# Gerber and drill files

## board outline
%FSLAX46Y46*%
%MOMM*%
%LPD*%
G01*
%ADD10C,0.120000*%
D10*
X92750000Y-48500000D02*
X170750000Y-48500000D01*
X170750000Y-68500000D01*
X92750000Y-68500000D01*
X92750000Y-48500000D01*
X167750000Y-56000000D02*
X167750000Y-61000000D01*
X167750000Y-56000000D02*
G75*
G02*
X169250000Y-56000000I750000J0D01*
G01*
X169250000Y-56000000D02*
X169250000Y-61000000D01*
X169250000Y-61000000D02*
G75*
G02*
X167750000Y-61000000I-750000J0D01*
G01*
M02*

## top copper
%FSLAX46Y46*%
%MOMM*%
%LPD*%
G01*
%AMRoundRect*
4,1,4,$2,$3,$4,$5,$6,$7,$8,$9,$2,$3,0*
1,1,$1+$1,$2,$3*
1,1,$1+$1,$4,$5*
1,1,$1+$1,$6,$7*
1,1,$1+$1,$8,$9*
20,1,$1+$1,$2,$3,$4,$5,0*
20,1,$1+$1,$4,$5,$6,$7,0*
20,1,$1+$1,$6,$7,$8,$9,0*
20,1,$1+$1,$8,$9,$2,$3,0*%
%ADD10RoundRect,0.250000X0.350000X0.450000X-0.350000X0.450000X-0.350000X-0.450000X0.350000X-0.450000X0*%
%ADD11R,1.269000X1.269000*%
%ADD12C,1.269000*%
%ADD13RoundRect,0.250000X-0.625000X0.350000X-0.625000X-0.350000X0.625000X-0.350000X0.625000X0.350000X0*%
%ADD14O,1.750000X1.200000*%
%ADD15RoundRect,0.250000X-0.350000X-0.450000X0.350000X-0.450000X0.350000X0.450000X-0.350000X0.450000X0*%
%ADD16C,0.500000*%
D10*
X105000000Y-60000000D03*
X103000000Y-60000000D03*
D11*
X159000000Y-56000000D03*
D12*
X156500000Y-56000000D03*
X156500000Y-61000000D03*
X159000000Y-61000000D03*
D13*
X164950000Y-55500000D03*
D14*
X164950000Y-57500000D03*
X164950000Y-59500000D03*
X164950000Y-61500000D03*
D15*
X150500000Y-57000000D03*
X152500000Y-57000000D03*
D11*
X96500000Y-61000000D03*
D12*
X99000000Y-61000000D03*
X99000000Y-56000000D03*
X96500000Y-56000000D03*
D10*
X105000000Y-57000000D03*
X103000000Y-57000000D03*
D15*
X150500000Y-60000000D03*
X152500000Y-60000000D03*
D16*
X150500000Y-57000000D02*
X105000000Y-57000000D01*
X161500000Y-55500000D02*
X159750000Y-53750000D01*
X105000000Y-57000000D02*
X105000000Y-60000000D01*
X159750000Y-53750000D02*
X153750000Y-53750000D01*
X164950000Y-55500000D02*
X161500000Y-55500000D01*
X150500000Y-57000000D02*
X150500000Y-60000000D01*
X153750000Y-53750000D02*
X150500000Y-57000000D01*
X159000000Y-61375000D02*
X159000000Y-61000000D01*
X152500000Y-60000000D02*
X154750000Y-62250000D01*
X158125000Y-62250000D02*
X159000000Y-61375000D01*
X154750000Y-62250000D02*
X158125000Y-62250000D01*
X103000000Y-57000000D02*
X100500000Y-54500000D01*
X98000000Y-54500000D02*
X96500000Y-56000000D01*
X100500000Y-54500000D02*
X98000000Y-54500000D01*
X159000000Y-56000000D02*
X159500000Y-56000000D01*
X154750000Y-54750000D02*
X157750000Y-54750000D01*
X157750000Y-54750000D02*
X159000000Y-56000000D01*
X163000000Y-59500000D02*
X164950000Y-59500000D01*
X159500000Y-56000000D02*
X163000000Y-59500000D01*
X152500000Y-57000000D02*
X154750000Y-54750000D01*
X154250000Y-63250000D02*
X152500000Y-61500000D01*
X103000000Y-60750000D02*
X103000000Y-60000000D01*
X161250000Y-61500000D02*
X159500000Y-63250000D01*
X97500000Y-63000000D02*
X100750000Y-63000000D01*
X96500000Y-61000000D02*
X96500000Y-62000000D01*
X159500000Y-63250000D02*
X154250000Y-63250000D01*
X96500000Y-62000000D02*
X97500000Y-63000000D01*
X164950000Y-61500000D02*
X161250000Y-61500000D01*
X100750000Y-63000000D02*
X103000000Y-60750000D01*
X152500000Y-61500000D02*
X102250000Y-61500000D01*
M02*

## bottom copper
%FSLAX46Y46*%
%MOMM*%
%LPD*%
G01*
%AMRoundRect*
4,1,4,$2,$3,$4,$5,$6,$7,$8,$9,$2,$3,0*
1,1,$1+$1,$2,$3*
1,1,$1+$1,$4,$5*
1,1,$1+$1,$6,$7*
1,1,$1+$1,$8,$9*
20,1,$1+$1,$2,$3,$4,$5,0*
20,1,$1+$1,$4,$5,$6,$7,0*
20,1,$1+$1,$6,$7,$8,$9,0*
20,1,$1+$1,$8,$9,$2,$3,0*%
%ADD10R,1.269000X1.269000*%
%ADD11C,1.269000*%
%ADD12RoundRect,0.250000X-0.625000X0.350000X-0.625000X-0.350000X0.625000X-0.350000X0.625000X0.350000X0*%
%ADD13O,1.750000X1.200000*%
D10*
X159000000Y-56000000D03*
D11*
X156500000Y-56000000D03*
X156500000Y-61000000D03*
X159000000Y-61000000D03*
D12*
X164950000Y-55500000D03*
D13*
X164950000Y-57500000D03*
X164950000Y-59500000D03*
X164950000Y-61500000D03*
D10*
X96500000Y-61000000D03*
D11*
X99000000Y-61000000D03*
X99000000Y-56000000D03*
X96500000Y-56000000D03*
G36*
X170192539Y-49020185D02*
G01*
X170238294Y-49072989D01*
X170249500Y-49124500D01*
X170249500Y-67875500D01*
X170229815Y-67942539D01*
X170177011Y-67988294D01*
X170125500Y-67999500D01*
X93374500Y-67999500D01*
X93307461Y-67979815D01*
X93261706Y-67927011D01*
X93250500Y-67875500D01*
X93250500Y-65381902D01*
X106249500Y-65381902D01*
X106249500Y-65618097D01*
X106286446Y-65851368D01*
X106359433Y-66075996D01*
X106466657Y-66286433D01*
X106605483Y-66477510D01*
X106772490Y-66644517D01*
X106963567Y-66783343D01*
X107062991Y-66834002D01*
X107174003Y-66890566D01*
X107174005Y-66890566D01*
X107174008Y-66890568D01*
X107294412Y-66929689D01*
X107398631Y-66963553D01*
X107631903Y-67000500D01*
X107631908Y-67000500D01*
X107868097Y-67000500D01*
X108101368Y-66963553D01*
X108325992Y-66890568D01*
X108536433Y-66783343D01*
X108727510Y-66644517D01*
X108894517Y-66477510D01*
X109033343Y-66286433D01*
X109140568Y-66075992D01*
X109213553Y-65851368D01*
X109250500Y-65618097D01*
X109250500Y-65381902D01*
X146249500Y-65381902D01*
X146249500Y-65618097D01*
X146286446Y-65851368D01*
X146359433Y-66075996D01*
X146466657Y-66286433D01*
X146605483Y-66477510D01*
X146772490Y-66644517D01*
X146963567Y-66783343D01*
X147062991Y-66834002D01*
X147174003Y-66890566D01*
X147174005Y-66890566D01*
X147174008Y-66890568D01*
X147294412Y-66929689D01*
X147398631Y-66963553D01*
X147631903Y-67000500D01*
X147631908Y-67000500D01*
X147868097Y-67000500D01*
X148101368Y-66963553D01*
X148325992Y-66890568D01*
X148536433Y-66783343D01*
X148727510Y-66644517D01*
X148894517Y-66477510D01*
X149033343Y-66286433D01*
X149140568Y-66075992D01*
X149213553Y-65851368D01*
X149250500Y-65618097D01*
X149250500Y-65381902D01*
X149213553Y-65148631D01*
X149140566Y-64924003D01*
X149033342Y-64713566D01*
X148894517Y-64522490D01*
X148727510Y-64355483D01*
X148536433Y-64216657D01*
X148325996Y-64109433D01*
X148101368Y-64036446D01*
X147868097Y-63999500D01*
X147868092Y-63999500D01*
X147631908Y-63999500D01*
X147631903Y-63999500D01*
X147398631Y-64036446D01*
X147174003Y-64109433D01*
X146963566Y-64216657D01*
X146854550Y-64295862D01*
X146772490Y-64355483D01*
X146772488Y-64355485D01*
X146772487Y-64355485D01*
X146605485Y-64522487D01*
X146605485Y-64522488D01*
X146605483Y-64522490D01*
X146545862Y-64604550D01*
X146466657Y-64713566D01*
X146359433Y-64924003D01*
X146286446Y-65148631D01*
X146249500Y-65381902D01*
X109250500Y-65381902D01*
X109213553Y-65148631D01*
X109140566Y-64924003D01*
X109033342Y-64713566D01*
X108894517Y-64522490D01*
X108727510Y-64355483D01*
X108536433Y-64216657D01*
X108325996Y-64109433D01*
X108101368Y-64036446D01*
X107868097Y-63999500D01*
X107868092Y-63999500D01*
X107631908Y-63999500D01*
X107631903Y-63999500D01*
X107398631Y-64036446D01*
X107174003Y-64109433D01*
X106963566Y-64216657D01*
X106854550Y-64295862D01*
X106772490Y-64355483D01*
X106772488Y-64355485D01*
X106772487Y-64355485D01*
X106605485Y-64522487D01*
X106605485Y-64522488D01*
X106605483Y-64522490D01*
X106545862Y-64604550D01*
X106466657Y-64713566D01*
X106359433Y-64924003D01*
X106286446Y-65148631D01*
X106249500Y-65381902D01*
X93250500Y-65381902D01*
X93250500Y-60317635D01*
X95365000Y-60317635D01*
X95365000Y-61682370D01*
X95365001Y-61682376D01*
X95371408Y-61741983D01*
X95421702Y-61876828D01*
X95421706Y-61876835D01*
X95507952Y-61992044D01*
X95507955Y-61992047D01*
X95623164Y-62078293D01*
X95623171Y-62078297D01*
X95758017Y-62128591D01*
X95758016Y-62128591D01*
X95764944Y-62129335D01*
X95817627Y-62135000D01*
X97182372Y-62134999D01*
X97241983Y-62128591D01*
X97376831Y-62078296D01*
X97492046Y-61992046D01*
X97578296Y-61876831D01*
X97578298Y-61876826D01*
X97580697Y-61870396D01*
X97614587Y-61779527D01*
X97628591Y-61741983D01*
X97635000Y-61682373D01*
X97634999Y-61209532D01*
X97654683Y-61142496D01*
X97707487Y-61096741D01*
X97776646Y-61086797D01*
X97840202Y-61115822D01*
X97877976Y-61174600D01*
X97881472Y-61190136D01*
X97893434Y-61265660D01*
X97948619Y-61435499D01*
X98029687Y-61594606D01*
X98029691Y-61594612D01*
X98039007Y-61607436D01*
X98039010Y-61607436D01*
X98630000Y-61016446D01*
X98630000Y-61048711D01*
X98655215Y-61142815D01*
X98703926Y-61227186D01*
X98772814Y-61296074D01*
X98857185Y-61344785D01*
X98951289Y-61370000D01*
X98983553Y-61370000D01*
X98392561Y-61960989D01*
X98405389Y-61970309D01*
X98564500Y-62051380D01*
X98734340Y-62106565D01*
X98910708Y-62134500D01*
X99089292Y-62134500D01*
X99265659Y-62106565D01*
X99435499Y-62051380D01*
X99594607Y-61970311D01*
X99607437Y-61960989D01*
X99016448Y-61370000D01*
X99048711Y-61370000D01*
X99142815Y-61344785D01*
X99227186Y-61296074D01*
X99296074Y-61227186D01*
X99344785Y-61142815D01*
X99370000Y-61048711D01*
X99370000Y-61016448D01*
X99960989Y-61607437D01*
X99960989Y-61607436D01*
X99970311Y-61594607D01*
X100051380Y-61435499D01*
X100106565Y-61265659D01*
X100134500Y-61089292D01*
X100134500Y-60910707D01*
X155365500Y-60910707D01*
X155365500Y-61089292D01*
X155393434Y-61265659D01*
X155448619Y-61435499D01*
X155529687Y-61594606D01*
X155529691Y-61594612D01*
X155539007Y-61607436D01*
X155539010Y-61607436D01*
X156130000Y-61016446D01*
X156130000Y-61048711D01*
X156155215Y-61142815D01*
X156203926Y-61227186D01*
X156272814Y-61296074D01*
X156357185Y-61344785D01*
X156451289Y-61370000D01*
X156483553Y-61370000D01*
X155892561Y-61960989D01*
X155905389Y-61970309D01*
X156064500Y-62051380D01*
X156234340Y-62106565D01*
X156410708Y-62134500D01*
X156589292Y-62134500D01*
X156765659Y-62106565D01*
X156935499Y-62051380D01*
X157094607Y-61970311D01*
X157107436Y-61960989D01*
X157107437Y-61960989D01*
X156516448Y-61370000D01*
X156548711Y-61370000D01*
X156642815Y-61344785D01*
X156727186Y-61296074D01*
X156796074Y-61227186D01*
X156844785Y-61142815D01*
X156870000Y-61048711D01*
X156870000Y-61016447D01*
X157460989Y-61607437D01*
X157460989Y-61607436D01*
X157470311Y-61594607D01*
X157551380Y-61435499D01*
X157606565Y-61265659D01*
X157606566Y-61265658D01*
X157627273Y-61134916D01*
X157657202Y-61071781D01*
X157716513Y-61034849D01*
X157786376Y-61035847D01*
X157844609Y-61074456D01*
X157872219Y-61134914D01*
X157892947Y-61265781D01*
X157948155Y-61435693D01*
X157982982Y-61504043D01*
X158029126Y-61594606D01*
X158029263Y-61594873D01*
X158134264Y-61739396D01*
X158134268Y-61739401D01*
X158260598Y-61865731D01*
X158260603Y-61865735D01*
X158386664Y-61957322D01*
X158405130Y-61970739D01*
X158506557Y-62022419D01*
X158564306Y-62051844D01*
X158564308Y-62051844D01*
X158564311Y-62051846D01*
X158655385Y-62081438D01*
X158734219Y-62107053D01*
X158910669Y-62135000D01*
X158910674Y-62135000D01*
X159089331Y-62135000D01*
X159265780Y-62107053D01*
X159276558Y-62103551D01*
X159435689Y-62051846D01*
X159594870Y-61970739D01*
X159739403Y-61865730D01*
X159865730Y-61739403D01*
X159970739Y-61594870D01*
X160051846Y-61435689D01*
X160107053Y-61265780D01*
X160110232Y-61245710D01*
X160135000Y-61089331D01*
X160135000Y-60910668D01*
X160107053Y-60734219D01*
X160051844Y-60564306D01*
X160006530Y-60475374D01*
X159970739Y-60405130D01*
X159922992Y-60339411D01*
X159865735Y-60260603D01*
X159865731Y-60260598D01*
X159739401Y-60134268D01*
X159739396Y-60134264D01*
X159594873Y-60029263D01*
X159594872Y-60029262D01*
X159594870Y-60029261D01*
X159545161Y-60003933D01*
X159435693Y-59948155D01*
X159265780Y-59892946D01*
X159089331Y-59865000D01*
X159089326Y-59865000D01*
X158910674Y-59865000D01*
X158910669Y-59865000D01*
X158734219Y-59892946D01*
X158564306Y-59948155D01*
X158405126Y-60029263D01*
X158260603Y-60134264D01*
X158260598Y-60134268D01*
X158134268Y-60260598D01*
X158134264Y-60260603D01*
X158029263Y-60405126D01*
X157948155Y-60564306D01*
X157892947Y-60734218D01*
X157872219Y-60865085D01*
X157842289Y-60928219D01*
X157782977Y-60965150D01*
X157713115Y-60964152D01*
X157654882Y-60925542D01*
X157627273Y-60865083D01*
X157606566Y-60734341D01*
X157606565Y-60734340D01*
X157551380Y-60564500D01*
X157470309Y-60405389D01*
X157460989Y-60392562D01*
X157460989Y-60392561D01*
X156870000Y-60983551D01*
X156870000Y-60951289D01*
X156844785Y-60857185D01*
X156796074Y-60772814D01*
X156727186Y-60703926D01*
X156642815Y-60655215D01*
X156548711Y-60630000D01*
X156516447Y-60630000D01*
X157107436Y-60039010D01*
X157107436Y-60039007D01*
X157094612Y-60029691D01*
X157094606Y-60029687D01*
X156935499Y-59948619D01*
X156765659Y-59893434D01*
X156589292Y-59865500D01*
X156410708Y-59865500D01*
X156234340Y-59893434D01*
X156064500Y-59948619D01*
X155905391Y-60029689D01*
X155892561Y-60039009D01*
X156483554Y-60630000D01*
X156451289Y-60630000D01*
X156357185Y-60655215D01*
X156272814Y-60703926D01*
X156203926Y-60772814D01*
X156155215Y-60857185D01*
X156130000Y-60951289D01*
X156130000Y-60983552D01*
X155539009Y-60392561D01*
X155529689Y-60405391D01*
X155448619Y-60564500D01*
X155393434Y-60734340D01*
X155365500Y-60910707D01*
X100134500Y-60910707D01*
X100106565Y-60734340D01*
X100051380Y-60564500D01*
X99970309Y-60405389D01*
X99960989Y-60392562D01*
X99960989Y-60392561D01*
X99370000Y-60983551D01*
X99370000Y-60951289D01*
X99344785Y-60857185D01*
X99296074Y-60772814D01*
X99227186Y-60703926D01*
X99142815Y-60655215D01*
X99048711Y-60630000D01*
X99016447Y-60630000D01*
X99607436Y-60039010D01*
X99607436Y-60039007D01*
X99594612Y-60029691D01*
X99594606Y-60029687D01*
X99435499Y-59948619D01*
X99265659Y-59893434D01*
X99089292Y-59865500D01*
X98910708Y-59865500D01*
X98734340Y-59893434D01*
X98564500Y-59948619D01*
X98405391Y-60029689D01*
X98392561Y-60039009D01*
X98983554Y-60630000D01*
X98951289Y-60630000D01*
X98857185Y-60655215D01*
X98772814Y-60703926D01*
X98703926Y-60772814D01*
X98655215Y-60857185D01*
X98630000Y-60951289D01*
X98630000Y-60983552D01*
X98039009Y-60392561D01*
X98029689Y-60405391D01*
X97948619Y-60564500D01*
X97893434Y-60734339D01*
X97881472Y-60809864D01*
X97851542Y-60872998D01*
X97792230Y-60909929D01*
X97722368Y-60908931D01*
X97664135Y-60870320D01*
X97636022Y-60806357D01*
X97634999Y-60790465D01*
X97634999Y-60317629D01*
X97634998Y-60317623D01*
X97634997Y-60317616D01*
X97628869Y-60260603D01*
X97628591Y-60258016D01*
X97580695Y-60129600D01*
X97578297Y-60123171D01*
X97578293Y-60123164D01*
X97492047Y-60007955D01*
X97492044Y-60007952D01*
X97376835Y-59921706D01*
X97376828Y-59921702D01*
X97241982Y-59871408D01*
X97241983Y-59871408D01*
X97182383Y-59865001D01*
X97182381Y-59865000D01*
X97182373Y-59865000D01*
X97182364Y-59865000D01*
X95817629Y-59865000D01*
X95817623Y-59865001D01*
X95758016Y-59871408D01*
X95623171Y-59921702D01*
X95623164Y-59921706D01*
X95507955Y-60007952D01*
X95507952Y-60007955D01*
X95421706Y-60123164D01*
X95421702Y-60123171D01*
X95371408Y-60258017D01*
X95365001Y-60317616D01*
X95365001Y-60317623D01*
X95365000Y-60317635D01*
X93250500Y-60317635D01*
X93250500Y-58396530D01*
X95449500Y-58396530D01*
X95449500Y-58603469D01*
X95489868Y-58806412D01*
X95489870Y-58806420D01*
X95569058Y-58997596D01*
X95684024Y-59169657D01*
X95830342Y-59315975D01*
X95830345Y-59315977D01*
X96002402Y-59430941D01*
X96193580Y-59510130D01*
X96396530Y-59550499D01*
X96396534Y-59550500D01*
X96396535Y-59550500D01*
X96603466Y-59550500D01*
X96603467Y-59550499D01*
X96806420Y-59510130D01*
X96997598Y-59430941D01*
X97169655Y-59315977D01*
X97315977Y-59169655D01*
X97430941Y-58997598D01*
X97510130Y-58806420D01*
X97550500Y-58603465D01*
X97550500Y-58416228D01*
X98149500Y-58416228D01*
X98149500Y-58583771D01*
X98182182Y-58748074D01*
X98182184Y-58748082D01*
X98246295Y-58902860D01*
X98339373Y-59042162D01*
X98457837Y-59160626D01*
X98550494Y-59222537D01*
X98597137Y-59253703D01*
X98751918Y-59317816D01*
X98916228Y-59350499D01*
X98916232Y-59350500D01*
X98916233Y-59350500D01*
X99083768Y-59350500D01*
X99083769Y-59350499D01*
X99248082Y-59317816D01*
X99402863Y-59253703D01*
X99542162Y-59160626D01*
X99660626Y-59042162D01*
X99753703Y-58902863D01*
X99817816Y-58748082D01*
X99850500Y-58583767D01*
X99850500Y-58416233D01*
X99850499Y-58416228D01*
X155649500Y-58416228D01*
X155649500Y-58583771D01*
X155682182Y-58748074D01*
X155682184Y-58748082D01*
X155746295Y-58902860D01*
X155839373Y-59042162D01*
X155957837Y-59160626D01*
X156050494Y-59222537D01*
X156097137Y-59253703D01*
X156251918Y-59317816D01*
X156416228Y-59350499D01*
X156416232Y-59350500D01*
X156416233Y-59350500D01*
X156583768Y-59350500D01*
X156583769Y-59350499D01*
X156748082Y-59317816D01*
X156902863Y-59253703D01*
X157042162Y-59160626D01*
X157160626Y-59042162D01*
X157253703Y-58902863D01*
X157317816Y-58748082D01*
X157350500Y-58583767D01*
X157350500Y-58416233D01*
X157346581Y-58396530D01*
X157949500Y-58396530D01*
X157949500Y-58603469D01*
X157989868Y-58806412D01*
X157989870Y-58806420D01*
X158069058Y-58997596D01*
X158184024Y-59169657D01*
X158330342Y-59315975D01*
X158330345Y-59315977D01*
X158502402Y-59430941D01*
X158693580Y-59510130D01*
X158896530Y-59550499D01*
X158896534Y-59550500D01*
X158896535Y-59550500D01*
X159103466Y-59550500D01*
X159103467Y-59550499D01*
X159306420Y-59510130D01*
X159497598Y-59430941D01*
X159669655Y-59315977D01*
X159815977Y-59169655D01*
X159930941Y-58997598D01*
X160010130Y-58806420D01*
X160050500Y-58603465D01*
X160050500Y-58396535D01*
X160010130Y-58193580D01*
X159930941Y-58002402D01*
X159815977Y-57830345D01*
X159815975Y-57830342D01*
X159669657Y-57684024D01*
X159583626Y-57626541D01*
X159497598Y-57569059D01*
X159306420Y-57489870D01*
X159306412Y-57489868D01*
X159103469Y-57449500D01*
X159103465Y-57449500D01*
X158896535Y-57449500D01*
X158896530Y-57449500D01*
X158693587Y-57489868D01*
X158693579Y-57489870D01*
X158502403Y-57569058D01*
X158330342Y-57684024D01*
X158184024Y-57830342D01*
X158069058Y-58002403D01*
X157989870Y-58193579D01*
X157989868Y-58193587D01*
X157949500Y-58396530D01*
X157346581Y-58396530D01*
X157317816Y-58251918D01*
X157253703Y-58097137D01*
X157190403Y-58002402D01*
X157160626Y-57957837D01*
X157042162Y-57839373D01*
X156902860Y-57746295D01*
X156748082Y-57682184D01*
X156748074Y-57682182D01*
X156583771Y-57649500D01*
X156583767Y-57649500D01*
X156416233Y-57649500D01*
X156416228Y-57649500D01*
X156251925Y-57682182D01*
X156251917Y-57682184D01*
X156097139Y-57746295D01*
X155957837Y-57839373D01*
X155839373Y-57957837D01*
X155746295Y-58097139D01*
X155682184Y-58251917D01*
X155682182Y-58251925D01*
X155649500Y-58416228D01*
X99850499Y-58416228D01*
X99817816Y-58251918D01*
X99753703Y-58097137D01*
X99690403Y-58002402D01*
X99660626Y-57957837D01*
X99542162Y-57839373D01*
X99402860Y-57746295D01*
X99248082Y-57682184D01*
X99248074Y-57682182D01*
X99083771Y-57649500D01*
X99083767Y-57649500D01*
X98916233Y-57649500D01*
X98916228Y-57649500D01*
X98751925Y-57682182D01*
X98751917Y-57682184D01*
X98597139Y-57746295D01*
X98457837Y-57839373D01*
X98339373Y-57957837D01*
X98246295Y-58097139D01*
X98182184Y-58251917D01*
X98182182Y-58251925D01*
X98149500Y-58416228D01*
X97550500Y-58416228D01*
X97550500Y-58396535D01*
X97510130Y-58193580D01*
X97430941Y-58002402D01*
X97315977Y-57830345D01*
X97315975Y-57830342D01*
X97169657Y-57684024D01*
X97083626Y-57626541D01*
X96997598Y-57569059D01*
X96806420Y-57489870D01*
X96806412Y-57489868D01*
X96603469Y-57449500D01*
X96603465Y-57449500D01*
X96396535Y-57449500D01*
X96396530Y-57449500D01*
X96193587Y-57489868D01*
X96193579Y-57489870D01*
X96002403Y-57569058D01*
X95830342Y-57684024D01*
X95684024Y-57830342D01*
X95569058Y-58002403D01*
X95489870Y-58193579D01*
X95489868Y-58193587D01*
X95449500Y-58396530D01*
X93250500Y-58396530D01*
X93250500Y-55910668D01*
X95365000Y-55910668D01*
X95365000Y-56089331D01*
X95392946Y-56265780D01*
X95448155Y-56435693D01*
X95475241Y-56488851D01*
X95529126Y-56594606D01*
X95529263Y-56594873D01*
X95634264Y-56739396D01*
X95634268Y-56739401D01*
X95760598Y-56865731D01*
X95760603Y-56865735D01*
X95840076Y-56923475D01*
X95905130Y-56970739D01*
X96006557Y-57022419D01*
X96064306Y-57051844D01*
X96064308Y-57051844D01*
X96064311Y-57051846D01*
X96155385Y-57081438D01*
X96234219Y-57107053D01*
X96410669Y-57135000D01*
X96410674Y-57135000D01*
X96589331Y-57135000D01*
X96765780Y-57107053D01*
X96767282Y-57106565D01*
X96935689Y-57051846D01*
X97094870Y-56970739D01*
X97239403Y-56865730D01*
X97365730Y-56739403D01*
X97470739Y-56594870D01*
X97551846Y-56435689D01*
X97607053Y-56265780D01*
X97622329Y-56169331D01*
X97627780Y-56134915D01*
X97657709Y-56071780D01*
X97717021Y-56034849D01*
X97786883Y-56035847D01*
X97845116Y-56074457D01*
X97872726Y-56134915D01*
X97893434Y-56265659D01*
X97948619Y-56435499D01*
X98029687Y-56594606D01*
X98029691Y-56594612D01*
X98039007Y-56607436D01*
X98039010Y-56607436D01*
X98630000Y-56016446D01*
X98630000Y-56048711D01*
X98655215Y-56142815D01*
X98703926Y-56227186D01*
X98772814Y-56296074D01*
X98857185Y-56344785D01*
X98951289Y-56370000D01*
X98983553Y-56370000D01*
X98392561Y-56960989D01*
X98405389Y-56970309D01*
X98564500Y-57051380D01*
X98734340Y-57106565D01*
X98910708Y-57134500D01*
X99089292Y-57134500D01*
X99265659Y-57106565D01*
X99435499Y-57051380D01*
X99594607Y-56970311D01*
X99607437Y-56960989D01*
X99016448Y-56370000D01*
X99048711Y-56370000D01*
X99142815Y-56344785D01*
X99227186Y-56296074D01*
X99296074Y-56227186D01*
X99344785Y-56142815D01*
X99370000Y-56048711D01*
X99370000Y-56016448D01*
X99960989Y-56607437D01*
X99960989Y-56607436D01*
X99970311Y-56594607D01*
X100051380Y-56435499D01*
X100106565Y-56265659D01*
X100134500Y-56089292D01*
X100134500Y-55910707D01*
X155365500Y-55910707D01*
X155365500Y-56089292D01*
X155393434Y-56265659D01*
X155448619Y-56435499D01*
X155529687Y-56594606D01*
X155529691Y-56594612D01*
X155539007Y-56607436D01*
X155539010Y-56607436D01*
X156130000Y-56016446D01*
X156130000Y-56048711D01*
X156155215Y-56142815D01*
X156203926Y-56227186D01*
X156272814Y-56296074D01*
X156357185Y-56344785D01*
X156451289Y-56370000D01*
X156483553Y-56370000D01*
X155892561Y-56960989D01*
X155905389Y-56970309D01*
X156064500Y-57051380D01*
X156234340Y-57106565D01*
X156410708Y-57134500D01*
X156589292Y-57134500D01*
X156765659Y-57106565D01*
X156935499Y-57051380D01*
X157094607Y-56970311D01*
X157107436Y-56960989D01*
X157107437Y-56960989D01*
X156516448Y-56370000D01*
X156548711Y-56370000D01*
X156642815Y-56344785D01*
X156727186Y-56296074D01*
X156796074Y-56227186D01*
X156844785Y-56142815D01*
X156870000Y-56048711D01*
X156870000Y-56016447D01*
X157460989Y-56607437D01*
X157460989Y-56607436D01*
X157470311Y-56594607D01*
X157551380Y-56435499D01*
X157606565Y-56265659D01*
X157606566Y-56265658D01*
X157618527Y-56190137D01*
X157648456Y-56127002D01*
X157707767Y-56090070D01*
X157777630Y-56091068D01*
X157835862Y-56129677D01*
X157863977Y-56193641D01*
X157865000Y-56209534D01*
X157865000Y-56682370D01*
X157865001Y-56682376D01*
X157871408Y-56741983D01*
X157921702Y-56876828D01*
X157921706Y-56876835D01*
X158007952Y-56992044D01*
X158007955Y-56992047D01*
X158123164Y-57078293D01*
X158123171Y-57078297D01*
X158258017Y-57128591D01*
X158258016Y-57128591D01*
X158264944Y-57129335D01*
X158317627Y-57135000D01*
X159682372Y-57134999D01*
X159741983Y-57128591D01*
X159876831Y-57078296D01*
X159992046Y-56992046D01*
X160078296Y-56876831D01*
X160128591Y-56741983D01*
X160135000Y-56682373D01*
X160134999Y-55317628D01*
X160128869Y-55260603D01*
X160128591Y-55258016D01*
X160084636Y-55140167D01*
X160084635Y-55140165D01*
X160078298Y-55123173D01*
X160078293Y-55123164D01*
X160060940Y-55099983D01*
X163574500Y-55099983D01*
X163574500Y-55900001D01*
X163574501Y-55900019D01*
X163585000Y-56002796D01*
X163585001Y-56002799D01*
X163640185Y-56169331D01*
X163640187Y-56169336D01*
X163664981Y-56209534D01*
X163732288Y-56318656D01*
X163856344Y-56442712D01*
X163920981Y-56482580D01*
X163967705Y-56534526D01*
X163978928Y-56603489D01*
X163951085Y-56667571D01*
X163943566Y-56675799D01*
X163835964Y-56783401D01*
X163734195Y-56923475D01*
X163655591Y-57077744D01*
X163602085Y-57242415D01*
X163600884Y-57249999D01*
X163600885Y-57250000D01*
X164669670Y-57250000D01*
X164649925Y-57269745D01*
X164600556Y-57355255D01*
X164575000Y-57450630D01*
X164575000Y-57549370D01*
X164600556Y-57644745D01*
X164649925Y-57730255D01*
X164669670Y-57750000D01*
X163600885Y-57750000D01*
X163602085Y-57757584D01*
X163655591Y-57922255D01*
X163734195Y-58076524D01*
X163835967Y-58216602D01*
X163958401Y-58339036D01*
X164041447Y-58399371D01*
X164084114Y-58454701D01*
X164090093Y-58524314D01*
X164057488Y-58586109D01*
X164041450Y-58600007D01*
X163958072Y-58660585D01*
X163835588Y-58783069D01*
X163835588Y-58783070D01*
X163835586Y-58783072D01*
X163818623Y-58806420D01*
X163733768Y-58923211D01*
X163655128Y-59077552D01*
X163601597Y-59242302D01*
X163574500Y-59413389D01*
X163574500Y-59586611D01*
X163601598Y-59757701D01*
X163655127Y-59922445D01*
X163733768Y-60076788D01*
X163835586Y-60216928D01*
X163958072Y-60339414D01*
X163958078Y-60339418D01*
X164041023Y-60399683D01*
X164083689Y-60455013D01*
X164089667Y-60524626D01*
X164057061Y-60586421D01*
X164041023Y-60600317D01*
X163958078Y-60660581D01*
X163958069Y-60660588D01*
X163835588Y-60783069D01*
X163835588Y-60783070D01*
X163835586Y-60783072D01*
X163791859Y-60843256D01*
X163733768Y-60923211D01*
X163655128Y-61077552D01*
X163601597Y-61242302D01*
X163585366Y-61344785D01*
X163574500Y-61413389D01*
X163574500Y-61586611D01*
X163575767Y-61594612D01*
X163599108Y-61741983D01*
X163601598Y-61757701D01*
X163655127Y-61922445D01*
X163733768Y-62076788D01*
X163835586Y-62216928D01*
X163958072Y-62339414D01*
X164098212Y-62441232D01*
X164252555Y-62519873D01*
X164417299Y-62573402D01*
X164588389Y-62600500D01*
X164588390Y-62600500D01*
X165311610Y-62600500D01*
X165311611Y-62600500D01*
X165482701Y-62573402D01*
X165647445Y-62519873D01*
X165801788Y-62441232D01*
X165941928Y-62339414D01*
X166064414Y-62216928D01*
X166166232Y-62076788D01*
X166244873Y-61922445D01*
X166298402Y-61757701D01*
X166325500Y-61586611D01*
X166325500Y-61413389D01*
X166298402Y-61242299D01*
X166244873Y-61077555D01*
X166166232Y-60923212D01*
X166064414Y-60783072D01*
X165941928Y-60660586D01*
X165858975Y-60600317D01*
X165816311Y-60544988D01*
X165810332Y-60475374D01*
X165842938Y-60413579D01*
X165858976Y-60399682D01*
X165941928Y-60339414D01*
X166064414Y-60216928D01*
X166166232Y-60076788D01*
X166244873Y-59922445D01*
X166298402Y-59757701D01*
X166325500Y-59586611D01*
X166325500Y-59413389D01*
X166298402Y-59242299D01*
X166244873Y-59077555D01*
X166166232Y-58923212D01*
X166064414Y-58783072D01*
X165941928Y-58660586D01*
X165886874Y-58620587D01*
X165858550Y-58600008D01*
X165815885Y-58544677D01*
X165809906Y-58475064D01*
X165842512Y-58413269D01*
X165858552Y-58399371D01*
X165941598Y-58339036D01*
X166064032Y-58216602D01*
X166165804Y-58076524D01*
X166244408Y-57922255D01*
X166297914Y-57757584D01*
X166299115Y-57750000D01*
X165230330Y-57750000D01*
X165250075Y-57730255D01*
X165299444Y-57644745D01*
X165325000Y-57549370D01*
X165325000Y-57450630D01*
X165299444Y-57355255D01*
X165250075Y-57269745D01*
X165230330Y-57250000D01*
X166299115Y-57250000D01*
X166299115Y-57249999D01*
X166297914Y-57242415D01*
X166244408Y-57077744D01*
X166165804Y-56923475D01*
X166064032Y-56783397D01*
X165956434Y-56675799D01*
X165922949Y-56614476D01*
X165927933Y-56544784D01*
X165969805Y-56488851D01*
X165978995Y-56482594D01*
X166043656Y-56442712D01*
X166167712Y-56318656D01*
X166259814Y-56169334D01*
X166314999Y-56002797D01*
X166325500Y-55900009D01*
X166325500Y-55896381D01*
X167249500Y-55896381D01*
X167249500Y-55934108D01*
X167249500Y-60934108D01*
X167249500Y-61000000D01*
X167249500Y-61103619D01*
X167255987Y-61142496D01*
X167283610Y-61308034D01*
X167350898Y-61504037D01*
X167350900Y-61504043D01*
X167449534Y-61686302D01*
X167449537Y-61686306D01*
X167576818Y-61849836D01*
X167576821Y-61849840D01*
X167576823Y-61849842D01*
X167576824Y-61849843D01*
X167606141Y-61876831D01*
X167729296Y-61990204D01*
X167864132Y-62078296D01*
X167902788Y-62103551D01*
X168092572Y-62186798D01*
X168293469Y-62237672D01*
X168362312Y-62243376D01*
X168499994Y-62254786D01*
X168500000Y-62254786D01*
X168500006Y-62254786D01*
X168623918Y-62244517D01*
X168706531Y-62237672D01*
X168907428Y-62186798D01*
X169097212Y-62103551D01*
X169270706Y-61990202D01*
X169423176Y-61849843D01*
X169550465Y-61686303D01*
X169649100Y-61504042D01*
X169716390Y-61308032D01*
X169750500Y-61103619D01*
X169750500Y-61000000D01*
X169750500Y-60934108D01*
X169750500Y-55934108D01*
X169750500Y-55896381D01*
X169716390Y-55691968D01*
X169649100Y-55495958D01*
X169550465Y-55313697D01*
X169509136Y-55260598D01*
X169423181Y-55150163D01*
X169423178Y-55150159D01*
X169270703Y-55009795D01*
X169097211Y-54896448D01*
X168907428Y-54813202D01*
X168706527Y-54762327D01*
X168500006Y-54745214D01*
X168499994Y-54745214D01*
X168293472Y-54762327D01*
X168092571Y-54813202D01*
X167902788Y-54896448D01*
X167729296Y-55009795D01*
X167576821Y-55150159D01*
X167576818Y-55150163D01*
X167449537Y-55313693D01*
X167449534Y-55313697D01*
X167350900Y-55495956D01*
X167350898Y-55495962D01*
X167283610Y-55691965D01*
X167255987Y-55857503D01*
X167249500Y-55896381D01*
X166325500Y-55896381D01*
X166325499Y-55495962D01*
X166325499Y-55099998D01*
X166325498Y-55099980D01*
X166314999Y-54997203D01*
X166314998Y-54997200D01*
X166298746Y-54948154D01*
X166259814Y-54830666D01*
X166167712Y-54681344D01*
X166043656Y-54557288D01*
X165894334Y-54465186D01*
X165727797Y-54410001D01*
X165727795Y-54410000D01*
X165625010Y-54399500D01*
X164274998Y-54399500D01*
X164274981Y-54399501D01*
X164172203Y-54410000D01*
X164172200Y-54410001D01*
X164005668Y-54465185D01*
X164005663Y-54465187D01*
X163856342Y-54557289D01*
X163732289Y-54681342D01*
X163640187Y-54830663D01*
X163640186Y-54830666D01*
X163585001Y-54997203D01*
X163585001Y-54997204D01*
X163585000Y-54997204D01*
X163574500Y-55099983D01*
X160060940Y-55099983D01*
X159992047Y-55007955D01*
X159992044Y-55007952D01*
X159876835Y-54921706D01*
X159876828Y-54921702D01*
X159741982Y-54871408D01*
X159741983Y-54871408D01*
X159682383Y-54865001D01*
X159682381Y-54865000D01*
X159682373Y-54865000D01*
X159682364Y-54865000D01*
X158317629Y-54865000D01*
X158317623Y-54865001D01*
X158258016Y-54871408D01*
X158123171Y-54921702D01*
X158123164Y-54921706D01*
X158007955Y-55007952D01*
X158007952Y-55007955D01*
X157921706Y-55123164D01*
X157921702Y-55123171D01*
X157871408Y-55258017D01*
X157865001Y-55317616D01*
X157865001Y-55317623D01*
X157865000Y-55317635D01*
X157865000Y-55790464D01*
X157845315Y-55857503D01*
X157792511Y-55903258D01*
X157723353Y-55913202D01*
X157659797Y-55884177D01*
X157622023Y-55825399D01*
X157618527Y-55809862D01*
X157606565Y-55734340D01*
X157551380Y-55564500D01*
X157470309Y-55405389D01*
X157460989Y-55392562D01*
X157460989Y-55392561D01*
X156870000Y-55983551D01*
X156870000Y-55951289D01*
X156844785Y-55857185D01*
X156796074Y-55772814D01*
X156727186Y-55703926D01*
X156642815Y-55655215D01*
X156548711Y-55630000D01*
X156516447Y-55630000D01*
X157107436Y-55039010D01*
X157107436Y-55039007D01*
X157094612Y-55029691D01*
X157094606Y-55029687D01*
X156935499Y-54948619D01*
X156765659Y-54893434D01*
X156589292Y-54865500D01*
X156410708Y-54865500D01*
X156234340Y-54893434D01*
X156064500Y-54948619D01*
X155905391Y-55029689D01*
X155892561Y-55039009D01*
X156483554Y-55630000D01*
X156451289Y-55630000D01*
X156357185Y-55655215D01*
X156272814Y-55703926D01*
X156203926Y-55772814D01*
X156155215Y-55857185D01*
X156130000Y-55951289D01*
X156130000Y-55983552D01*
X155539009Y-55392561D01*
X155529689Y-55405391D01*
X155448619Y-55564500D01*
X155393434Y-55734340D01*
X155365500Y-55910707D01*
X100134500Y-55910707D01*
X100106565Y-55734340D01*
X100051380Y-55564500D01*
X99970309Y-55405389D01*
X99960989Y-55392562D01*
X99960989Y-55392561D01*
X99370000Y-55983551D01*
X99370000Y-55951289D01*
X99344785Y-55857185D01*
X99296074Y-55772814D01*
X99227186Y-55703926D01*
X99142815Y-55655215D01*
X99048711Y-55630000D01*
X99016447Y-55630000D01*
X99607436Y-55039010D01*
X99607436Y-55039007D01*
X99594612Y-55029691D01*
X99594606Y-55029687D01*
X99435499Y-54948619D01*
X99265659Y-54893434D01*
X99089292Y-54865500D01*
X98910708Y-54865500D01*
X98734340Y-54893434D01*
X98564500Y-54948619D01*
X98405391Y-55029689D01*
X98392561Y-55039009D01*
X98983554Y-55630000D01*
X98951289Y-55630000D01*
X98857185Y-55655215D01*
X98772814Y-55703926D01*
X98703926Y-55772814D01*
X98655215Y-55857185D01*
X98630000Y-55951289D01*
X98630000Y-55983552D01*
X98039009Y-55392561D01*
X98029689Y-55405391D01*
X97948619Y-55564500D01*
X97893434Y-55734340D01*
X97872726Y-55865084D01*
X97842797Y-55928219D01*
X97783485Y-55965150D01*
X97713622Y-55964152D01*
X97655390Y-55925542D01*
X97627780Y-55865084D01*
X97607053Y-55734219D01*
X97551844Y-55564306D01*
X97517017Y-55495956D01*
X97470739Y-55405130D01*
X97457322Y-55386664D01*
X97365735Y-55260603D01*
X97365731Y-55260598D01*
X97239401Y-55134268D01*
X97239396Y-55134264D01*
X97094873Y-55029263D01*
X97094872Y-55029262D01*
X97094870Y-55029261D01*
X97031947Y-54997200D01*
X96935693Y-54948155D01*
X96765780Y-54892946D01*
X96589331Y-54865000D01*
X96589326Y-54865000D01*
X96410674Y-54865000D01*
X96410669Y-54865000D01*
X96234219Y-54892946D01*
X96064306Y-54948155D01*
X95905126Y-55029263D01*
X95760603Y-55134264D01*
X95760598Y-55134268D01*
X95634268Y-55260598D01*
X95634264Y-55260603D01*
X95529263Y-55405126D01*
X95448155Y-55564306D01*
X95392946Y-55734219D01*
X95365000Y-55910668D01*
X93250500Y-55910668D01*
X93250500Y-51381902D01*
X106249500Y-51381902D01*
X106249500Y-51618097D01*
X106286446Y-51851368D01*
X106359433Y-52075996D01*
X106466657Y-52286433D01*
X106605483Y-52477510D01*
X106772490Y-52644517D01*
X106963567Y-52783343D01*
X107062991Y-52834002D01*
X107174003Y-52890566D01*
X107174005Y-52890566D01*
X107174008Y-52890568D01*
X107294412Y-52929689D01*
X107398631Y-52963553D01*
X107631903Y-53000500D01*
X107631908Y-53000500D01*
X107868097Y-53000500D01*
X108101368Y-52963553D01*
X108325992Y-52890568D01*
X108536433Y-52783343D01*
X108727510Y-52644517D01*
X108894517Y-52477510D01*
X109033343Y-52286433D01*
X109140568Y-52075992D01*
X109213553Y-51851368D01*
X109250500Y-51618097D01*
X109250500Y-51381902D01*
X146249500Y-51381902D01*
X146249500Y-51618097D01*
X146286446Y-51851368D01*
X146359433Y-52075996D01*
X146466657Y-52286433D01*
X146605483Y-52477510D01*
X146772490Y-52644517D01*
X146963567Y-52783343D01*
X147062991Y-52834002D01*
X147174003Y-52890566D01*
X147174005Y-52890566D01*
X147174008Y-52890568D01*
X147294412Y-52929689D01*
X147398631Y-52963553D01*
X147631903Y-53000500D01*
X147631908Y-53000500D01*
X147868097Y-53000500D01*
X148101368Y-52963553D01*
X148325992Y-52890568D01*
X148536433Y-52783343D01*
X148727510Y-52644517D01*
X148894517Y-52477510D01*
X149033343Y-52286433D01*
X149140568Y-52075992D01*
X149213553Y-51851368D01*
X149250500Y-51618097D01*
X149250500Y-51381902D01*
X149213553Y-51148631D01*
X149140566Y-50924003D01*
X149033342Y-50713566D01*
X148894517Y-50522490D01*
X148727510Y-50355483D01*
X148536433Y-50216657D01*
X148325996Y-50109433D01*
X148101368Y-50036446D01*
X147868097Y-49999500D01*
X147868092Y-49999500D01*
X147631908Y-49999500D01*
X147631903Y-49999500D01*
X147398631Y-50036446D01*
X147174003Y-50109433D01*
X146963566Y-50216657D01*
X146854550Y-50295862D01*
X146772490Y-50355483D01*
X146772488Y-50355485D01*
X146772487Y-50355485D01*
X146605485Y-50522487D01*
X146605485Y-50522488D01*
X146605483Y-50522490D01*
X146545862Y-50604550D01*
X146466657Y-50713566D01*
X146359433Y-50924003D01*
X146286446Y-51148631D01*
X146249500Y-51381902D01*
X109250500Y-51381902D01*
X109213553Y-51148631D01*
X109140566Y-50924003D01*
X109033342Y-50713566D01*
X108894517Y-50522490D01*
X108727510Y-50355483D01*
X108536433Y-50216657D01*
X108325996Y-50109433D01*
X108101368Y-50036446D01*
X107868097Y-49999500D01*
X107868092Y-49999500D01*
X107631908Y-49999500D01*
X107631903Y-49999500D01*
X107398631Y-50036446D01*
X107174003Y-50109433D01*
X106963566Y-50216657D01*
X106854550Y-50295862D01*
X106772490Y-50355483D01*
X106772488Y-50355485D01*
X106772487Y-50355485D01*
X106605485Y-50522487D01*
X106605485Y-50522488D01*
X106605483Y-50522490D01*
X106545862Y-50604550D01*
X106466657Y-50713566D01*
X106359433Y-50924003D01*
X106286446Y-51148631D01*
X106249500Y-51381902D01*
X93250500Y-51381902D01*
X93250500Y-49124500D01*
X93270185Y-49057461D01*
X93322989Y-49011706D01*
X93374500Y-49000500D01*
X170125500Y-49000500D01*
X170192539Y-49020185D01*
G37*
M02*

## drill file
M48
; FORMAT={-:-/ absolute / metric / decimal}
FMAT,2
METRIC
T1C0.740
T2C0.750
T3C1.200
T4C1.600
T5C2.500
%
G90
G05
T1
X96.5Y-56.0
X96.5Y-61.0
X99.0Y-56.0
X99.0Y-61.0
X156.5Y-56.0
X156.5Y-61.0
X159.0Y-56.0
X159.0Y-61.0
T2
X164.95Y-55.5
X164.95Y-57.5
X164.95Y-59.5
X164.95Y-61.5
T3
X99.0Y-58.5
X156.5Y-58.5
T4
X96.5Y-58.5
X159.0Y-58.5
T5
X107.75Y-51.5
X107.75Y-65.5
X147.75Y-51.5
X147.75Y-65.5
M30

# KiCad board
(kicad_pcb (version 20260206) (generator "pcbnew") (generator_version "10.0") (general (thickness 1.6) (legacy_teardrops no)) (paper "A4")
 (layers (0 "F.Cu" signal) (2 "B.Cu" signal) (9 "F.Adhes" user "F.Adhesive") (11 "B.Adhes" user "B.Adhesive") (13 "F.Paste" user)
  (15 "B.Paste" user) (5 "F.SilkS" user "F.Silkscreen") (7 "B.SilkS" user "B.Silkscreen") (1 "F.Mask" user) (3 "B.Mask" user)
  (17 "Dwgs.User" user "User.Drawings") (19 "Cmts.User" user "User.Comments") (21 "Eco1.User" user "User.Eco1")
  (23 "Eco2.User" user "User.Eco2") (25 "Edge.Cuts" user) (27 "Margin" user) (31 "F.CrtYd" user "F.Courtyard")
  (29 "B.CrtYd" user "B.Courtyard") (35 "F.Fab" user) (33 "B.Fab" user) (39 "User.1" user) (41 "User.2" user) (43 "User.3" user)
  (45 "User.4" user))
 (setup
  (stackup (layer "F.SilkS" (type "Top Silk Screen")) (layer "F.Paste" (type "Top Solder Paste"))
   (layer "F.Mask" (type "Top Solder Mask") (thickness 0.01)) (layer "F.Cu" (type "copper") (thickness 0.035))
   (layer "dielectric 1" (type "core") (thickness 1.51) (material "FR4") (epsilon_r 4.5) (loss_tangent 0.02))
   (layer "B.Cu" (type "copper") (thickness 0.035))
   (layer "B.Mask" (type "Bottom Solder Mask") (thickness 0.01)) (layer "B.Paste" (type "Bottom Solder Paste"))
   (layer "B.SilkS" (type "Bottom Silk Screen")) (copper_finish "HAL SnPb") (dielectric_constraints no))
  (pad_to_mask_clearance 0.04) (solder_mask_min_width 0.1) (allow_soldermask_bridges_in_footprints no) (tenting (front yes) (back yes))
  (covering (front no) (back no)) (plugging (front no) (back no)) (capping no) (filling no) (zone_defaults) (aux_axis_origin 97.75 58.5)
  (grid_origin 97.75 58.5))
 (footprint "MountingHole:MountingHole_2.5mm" (layer "F.Cu") (at 107.75 51.5)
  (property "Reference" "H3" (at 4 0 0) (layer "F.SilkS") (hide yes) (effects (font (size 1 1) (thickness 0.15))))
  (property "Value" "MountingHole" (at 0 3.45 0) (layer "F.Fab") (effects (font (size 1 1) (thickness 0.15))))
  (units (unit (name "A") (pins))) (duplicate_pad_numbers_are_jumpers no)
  (pad "" np_thru_hole circle (at 0 0) (size 2.5 2.5) (drill 2.5) (layers "*.Cu" "*.Mask")))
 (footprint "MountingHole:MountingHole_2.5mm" (layer "F.Cu") (at 107.75 65.5)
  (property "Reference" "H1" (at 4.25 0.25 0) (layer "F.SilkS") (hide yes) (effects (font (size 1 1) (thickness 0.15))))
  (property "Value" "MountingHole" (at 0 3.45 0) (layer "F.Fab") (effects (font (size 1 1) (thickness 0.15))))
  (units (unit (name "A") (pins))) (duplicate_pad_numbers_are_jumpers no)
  (pad "" np_thru_hole circle (at 0 0) (size 2.5 2.5) (drill 2.5) (layers "*.Cu" "*.Mask")))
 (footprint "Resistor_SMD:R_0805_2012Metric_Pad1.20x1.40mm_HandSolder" (layer "F.Cu") (at 104 60 180)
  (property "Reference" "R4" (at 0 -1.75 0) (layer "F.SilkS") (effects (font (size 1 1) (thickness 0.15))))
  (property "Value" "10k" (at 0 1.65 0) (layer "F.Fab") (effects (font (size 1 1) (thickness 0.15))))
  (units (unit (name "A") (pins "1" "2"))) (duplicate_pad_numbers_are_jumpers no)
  (pad "1" smd roundrect (at -1 0 180) (size 1.2 1.4) (layers "F.Cu" "F.Mask" "F.Paste") (roundrect_rratio 0.208333) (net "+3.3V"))
  (pad "2" smd roundrect (at 1 0 180) (size 1.2 1.4) (layers "F.Cu" "F.Mask" "F.Paste") (roundrect_rratio 0.208333) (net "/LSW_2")))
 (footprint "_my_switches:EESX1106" (layer "F.Cu") (at 159 56 -90)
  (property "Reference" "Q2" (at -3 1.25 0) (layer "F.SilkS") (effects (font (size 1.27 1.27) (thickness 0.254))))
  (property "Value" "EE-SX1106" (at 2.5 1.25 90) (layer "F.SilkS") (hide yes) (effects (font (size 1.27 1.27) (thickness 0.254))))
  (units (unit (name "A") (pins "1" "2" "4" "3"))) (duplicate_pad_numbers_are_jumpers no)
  (pad "" np_thru_hole circle (at 2.5 0 270) (size 1.6 1.6) (drill 1.6) (layers "*.Cu" "*.Mask"))
  (pad "" np_thru_hole circle (at 2.5 2.5 270) (size 1.2 1.2) (drill 1.2) (layers "*.Cu" "*.Mask"))
  (pad "1" thru_hole rect (at 0 0 270) (size 1.269 1.269) (drill 0.74) (layers "*.Cu" "*.Mask") (remove_unused_layers no) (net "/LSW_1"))
  (pad "2" thru_hole circle (at 0 2.5 270) (size 1.269 1.269) (drill 0.74) (layers "*.Cu" "*.Mask") (remove_unused_layers no) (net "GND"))
  (pad "3" thru_hole circle (at 5 2.5 270) (size 1.269 1.269) (drill 0.74) (layers "*.Cu" "*.Mask") (remove_unused_layers no) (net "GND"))
  (pad "4" thru_hole circle (at 5 0 270) (size 1.269 1.269) (drill 0.74) (layers "*.Cu" "*.Mask") (remove_unused_layers no)
   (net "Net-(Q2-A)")))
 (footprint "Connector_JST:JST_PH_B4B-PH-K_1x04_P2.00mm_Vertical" (layer "F.Cu") (at 164.95 55.5 -90)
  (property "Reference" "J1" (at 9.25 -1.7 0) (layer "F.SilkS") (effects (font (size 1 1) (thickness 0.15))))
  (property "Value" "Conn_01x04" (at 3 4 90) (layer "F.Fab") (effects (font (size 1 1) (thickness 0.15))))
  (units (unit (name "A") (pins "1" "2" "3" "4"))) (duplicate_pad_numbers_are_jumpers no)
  (pad "1" thru_hole roundrect (at 0 0 270) (size 1.2 1.75) (drill 0.75) (layers "*.Cu" "*.Mask") (remove_unused_layers no)
   (roundrect_rratio 0.208333) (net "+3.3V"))
  (pad "2" thru_hole oval (at 2 0 270) (size 1.2 1.75) (drill 0.75) (layers "*.Cu" "*.Mask") (remove_unused_layers no) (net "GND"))
  (pad "3" thru_hole oval (at 4 0 270) (size 1.2 1.75) (drill 0.75) (layers "*.Cu" "*.Mask") (remove_unused_layers no) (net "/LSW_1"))
  (pad "4" thru_hole oval (at 6 0 270) (size 1.2 1.75) (drill 0.75) (layers "*.Cu" "*.Mask") (remove_unused_layers no) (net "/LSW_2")))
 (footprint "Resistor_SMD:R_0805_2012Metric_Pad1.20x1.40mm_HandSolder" (layer "F.Cu") (at 151.5 57)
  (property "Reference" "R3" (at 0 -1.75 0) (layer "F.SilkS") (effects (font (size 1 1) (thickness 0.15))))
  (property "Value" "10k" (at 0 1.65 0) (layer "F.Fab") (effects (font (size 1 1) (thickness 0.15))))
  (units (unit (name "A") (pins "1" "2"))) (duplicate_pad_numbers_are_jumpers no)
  (pad "1" smd roundrect (at -1 0) (size 1.2 1.4) (layers "F.Cu" "F.Mask" "F.Paste") (roundrect_rratio 0.208333) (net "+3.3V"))
  (pad "2" smd roundrect (at 1 0) (size 1.2 1.4) (layers "F.Cu" "F.Mask" "F.Paste") (roundrect_rratio 0.208333) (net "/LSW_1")))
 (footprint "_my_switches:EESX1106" (layer "F.Cu") (at 96.5 61 90)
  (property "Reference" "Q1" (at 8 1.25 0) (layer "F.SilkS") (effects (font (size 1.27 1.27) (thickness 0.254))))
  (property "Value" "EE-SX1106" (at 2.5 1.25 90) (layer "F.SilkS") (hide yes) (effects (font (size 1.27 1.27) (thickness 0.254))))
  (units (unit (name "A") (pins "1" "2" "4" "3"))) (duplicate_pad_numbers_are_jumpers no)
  (pad "" np_thru_hole circle (at 2.5 0 90) (size 1.6 1.6) (drill 1.6) (layers "*.Cu" "*.Mask"))
  (pad "" np_thru_hole circle (at 2.5 2.5 90) (size 1.2 1.2) (drill 1.2) (layers "*.Cu" "*.Mask"))
  (pad "1" thru_hole rect (at 0 0 90) (size 1.269 1.269) (drill 0.74) (layers "*.Cu" "*.Mask") (remove_unused_layers no) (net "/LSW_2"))
  (pad "2" thru_hole circle (at 0 2.5 90) (size 1.269 1.269) (drill 0.74) (layers "*.Cu" "*.Mask") (remove_unused_layers no) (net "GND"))
  (pad "3" thru_hole circle (at 5 2.5 90) (size 1.269 1.269) (drill 0.74) (layers "*.Cu" "*.Mask") (remove_unused_layers no) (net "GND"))
  (pad "4" thru_hole circle (at 5 0 90) (size 1.269 1.269) (drill 0.74) (layers "*.Cu" "*.Mask") (remove_unused_layers no)
   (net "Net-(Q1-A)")))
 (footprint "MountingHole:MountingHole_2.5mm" (layer "F.Cu") (at 147.75 51.5)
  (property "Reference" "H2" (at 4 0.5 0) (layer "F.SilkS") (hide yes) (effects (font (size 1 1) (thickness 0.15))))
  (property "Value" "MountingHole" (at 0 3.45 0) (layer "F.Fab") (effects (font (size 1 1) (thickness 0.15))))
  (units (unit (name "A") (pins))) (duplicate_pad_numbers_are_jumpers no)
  (pad "" np_thru_hole circle (at 0 0) (size 2.5 2.5) (drill 2.5) (layers "*.Cu" "*.Mask")))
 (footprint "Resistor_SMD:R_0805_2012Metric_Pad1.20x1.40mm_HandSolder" (layer "F.Cu") (at 104 57 180)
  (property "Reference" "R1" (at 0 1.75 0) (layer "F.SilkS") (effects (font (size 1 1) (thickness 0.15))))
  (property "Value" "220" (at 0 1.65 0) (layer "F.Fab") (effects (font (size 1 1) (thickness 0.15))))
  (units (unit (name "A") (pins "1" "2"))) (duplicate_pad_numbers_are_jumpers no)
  (pad "1" smd roundrect (at -1 0 180) (size 1.2 1.4) (layers "F.Cu" "F.Mask" "F.Paste") (roundrect_rratio 0.208333) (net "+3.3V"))
  (pad "2" smd roundrect (at 1 0 180) (size 1.2 1.4) (layers "F.Cu" "F.Mask" "F.Paste") (roundrect_rratio 0.208333) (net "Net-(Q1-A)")))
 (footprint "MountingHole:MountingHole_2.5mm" (layer "F.Cu") (at 147.75 65.5)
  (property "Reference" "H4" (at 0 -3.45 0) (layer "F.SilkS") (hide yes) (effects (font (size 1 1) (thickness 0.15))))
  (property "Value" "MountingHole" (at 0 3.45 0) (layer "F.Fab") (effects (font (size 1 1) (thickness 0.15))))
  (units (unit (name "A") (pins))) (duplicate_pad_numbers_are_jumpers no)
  (pad "" np_thru_hole circle (at 0 0) (size 2.5 2.5) (drill 2.5) (layers "*.Cu" "*.Mask")))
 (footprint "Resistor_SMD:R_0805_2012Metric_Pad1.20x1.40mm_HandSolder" (layer "F.Cu") (at 151.5 60)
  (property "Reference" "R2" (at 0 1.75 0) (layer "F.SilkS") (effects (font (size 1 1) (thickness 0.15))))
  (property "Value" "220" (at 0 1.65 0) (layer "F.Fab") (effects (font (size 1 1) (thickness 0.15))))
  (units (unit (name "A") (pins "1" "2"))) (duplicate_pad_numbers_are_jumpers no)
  (pad "1" smd roundrect (at -1 0) (size 1.2 1.4) (layers "F.Cu" "F.Mask" "F.Paste") (roundrect_rratio 0.208333) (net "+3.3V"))
  (pad "2" smd roundrect (at 1 0) (size 1.2 1.4) (layers "F.Cu" "F.Mask" "F.Paste") (roundrect_rratio 0.208333) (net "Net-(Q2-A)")))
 (gr_rect (start 92.75 48.5) (end 170.75 68.5) (stroke (width 0.12) (type default)) (fill no) (layer "Edge.Cuts"))
 (gr_line (start 167.75 56) (end 167.75 61) (stroke (width 0.12) (type default)) (layer "Edge.Cuts"))
 (gr_arc (start 167.75 56) (mid 168.5 55.25) (end 169.25 56) (stroke (width 0.12) (type default)) (layer "Edge.Cuts"))
 (gr_line (start 169.25 56) (end 169.25 61) (stroke (width 0.12) (type default)) (layer "Edge.Cuts"))
 (gr_arc (start 169.25 61) (mid 168.5 61.75) (end 167.75 61) (stroke (width 0.12) (type default)) (layer "Edge.Cuts"))
 (segment (start 150.5 57) (end 105 57) (width 0.5) (layer "F.Cu") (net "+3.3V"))
 (segment (start 161.5 55.5) (end 159.75 53.75) (width 0.5) (layer "F.Cu") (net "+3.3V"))
 (segment (start 105 57) (end 105 60) (width 0.5) (layer "F.Cu") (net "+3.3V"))
 (segment (start 159.75 53.75) (end 153.75 53.75) (width 0.5) (layer "F.Cu") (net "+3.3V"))
 (segment (start 164.95 55.5) (end 161.5 55.5) (width 0.5) (layer "F.Cu") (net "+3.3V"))
 (segment (start 150.5 57) (end 150.5 60) (width 0.5) (layer "F.Cu") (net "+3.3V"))
 (segment (start 153.75 53.75) (end 150.5 57) (width 0.5) (layer "F.Cu") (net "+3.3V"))
 (segment (start 159 61.375) (end 159 61) (width 0.5) (layer "F.Cu") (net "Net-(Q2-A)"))
 (segment (start 152.5 60) (end 154.75 62.25) (width 0.5) (layer "F.Cu") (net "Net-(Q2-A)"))
 (segment (start 158.125 62.25) (end 159 61.375) (width 0.5) (layer "F.Cu") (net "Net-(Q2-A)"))
 (segment (start 154.75 62.25) (end 158.125 62.25) (width 0.5) (layer "F.Cu") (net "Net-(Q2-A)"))
 (segment (start 103 57) (end 100.5 54.5) (width 0.5) (layer "F.Cu") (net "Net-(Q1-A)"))
 (segment (start 98 54.5) (end 96.5 56) (width 0.5) (layer "F.Cu") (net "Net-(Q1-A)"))
 (segment (start 100.5 54.5) (end 98 54.5) (width 0.5) (layer "F.Cu") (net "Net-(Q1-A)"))
 (segment (start 159 56) (end 159.5 56) (width 0.5) (layer "F.Cu") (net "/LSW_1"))
 (segment (start 154.75 54.75) (end 157.75 54.75) (width 0.5) (layer "F.Cu") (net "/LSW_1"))
 (segment (start 157.75 54.75) (end 159 56) (width 0.5) (layer "F.Cu") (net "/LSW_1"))
 (segment (start 163 59.5) (end 164.95 59.5) (width 0.5) (layer "F.Cu") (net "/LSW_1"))
 (segment (start 159.5 56) (end 163 59.5) (width 0.5) (layer "F.Cu") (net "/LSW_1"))
 (segment (start 152.5 57) (end 154.75 54.75) (width 0.5) (layer "F.Cu") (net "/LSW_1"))
 (segment (start 154.25 63.25) (end 152.5 61.5) (width 0.5) (layer "F.Cu") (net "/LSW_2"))
 (segment (start 103 60.75) (end 103 60) (width 0.5) (layer "F.Cu") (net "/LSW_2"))
 (segment (start 161.25 61.5) (end 159.5 63.25) (width 0.5) (layer "F.Cu") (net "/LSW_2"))
 (segment (start 97.5 63) (end 100.75 63) (width 0.5) (layer "F.Cu") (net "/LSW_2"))
 (segment (start 96.5 61) (end 96.5 62) (width 0.5) (layer "F.Cu") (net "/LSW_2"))
 (segment (start 159.5 63.25) (end 154.25 63.25) (width 0.5) (layer "F.Cu") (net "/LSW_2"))
 (segment (start 96.5 62) (end 97.5 63) (width 0.5) (layer "F.Cu") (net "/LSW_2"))
 (segment (start 164.95 61.5) (end 161.25 61.5) (width 0.5) (layer "F.Cu") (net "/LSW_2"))
 (segment (start 100.75 63) (end 103 60.75) (width 0.5) (layer "F.Cu") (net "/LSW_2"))
 (segment (start 152.5 61.5) (end 102.25 61.5) (width 0.5) (layer "F.Cu") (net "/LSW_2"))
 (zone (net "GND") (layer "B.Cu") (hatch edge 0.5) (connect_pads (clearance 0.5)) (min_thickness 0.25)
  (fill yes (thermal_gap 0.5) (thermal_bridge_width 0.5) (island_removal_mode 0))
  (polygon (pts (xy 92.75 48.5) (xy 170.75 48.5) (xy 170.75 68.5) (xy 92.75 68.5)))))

